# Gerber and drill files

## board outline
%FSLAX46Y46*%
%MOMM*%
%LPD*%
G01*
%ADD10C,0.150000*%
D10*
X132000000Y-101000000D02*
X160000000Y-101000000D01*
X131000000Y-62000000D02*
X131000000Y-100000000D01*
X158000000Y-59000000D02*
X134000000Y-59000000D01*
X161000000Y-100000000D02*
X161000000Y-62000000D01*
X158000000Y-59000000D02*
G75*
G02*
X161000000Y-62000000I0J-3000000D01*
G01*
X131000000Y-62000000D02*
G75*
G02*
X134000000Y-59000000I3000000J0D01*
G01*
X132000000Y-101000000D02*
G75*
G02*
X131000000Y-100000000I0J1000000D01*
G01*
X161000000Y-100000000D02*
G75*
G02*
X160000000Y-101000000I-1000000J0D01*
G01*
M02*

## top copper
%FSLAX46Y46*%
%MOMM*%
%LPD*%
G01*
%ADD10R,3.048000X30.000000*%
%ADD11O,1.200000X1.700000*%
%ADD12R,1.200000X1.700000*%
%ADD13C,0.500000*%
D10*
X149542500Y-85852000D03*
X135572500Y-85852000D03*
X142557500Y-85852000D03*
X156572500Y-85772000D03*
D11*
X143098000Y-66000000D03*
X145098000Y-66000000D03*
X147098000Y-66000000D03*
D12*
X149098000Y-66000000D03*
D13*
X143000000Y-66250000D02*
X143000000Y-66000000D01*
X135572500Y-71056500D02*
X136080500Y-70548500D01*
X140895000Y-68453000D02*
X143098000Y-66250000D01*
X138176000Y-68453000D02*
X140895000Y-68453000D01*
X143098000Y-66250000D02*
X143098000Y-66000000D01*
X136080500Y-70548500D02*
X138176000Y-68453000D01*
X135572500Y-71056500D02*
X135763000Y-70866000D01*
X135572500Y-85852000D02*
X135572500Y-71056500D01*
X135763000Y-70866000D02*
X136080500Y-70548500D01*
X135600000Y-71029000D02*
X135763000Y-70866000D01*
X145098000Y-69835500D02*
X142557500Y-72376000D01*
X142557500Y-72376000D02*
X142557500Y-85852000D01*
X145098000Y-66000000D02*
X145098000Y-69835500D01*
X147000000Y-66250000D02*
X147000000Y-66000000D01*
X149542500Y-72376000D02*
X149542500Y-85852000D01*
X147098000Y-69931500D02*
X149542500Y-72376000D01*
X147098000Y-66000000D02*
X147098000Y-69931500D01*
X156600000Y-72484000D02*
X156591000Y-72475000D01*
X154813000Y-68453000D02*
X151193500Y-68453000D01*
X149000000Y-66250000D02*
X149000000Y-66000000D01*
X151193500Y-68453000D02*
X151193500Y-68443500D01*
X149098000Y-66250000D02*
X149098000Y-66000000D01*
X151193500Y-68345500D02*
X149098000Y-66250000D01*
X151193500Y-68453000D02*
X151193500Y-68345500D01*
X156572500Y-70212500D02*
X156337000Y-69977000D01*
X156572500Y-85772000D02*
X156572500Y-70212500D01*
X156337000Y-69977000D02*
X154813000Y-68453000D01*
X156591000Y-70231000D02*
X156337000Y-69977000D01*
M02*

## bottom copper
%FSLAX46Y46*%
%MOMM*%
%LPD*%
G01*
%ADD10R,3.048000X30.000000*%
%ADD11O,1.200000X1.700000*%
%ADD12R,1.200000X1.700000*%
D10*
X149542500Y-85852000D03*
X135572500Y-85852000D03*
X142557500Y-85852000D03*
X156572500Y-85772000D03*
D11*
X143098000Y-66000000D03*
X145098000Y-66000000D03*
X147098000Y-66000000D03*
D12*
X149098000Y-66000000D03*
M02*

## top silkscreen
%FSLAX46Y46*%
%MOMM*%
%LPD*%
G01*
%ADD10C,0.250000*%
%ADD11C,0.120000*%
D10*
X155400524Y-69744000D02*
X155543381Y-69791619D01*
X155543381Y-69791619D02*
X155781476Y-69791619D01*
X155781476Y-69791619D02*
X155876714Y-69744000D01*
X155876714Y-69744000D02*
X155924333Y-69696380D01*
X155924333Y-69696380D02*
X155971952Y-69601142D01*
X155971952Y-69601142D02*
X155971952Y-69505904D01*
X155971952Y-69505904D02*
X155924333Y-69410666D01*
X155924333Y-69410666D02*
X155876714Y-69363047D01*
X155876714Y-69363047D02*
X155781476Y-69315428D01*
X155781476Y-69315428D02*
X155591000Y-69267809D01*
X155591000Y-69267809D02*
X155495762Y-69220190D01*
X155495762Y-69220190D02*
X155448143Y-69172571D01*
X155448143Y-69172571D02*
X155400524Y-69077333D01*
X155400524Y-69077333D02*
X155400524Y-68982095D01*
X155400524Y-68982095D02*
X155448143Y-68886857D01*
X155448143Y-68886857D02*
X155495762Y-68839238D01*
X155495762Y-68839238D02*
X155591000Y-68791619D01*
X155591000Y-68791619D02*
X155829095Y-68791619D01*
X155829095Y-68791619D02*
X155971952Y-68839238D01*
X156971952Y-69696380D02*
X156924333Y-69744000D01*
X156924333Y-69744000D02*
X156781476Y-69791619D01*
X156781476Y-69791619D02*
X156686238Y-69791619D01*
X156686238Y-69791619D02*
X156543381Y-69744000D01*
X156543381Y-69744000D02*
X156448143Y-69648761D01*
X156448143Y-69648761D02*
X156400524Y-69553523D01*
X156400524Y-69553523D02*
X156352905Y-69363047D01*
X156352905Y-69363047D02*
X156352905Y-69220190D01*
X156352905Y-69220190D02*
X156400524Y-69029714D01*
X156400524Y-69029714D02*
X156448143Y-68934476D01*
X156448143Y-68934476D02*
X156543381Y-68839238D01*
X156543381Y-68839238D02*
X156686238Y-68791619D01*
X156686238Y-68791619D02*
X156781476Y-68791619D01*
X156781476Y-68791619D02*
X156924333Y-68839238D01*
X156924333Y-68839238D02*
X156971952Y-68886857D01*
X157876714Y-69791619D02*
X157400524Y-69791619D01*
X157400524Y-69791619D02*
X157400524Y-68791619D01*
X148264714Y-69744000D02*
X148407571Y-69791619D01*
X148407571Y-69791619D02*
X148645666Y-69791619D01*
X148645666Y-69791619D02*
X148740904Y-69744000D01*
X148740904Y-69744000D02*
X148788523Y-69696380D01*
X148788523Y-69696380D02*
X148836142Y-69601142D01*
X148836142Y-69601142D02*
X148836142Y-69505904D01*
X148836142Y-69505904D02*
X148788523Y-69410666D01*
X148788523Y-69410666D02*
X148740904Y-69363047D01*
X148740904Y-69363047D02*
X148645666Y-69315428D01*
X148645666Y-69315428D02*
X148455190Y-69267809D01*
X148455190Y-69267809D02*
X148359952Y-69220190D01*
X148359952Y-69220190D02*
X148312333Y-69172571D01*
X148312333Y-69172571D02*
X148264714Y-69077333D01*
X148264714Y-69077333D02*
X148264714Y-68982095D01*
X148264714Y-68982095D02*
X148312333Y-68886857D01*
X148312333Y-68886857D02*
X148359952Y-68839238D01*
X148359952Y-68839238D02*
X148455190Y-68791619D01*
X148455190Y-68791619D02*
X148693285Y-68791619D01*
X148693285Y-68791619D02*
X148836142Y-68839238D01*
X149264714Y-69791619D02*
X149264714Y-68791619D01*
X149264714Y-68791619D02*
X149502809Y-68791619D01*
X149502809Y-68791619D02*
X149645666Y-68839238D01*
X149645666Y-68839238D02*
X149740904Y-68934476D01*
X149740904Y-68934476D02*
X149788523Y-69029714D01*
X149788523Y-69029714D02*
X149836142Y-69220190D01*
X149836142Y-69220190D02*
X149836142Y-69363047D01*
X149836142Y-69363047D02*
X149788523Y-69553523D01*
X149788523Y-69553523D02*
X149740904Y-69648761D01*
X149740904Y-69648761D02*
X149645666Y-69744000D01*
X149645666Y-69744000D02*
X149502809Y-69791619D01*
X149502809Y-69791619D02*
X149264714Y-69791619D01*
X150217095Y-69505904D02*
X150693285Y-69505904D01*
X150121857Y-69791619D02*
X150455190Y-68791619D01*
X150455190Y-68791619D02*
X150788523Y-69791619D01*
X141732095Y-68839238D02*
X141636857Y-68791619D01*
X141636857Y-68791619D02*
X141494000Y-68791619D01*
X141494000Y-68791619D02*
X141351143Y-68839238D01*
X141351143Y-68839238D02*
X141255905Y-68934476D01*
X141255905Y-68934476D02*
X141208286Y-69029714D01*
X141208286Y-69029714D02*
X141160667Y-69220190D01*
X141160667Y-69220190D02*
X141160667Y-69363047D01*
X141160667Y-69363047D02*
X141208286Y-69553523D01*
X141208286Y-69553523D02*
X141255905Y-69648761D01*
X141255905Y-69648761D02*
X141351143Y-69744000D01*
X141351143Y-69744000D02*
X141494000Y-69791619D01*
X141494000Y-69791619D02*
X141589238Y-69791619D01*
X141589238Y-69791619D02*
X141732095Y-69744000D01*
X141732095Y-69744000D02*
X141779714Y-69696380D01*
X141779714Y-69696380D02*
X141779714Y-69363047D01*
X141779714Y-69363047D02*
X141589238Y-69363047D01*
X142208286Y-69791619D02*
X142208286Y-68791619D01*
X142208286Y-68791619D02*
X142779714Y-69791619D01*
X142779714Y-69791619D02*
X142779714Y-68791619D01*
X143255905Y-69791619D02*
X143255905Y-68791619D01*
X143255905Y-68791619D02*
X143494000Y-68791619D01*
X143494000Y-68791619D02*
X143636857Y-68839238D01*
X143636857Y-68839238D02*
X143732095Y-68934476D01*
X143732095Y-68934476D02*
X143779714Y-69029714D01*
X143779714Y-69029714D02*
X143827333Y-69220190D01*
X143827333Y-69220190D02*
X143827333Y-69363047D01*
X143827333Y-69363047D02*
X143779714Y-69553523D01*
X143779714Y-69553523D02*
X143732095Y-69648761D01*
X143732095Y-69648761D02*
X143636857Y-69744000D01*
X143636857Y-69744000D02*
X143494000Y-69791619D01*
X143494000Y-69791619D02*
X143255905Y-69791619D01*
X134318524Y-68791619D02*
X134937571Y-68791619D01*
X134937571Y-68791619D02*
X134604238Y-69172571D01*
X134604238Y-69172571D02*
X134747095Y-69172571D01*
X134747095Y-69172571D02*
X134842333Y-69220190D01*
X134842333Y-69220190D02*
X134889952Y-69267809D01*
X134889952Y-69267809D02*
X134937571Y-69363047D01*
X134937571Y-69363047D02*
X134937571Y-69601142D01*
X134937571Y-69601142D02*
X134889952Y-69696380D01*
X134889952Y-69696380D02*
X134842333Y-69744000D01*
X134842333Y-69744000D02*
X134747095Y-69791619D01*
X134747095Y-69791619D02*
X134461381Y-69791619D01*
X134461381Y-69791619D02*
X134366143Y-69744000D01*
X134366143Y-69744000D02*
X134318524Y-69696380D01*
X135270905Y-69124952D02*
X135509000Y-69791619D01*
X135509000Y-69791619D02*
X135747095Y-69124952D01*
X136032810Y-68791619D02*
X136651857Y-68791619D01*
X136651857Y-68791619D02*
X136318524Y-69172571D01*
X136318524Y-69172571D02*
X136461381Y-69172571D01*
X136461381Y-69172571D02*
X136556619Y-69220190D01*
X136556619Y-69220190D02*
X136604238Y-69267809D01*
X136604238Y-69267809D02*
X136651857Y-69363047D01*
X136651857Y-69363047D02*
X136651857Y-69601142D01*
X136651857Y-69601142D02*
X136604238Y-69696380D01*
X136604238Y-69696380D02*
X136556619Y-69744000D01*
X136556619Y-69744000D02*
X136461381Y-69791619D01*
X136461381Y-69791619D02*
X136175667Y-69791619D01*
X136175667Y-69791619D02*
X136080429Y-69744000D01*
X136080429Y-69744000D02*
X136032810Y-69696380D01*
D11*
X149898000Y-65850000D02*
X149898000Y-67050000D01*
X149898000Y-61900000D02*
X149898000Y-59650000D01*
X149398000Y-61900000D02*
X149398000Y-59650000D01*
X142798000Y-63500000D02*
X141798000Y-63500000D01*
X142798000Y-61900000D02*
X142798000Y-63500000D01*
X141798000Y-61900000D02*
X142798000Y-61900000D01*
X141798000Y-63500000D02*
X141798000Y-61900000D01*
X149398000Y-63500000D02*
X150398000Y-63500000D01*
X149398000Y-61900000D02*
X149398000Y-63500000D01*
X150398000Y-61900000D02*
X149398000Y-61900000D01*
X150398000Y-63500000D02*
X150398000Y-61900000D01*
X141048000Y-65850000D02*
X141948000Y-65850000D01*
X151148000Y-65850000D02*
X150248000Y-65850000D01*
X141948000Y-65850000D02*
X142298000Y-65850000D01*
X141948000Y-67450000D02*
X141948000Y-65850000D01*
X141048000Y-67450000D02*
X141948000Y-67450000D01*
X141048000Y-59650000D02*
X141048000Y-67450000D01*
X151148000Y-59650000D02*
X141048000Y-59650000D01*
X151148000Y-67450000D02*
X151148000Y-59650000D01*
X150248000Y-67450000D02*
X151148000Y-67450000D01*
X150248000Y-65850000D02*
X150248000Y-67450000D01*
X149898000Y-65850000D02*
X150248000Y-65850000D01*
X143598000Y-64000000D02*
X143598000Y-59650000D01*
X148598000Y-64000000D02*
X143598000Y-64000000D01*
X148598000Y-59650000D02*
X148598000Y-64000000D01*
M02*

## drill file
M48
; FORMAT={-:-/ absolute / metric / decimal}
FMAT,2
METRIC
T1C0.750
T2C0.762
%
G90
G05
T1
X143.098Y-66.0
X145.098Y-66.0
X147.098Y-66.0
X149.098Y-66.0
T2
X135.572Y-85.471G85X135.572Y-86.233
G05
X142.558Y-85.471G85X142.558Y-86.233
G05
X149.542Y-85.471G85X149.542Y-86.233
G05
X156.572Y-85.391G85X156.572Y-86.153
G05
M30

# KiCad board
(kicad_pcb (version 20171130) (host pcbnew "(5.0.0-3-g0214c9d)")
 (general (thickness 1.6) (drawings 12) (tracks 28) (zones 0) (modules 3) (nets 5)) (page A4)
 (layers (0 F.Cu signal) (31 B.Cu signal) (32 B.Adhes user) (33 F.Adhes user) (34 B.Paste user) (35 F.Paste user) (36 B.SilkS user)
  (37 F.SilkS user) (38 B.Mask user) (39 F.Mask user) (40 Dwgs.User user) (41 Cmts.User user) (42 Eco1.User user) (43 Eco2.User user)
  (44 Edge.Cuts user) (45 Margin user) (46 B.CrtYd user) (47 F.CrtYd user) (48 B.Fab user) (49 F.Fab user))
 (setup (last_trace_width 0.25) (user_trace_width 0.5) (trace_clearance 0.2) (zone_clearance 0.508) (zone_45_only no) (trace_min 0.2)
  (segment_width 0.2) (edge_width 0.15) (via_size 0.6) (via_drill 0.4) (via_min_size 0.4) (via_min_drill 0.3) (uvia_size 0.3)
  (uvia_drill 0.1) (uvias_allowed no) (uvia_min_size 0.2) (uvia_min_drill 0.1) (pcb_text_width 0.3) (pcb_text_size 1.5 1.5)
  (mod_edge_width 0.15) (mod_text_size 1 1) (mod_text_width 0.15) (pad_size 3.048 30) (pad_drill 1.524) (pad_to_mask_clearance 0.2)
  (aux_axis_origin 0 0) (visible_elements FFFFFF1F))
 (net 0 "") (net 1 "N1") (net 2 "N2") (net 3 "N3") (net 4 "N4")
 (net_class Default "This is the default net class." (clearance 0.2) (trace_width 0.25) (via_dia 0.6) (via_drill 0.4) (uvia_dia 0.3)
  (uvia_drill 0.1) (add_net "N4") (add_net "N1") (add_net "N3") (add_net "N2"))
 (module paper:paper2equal (layer B.Cu) (at 145.7325 70.612)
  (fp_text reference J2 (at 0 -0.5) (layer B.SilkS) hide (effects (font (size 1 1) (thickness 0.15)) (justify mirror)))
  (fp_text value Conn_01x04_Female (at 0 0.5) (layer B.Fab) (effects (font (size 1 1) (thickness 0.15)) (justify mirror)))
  (pad 3 thru_hole rect (at 3.81 15.24) (size 3.048 30) (drill oval 0.762 1.524) (layers *.Cu *.Mask) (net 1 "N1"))
  (pad 1 thru_hole rect (at -10.16 15.24) (size 3.048 30) (drill oval 0.762 1.524) (layers *.Cu *.Mask) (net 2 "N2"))
  (pad 2 thru_hole rect (at -3.175 15.24) (size 3.048 30) (drill oval 0.762 1.524) (layers *.Cu *.Mask) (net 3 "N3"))
  (pad 4 thru_hole rect (at 10.84 15.16) (size 3.048 30) (drill oval 0.762 1.524) (layers *.Cu *.Mask) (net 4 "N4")))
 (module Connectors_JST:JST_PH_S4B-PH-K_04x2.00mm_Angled (layer F.Cu) (at 149.098 66 180)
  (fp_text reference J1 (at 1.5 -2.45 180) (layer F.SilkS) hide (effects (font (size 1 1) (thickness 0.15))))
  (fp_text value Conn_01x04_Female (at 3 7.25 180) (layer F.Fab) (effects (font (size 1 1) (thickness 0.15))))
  (fp_line (start -0.8 0.15) (end -0.8 -1.05) (layer F.SilkS) (width 0.12))
  (fp_line (start -0.8 4.1) (end -0.8 6.35) (layer F.SilkS) (width 0.12))
  (fp_line (start -0.3 4.1) (end -0.3 6.35) (layer F.SilkS) (width 0.12))
  (fp_line (start 6.3 2.5) (end 7.3 2.5) (layer F.SilkS) (width 0.12))
  (fp_line (start 6.3 4.1) (end 6.3 2.5) (layer F.SilkS) (width 0.12))
  (fp_line (start 7.3 4.1) (end 6.3 4.1) (layer F.SilkS) (width 0.12))
  (fp_line (start 7.3 2.5) (end 7.3 4.1) (layer F.SilkS) (width 0.12))
  (fp_line (start -0.3 2.5) (end -1.3 2.5) (layer F.SilkS) (width 0.12))
  (fp_line (start -0.3 4.1) (end -0.3 2.5) (layer F.SilkS) (width 0.12))
  (fp_line (start -1.3 4.1) (end -0.3 4.1) (layer F.SilkS) (width 0.12))
  (fp_line (start -1.3 2.5) (end -1.3 4.1) (layer F.SilkS) (width 0.12))
  (fp_line (start 8.05 0.15) (end 7.15 0.15) (layer F.SilkS) (width 0.12))
  (fp_line (start -2.05 0.15) (end -1.15 0.15) (layer F.SilkS) (width 0.12))
  (fp_line (start 7.15 0.15) (end 6.8 0.15) (layer F.SilkS) (width 0.12))
  (fp_line (start 7.15 -1.45) (end 7.15 0.15) (layer F.SilkS) (width 0.12))
  (fp_line (start 8.05 -1.45) (end 7.15 -1.45) (layer F.SilkS) (width 0.12))
  (fp_line (start 8.05 6.35) (end 8.05 -1.45) (layer F.SilkS) (width 0.12))
  (fp_line (start -2.05 6.35) (end 8.05 6.35) (layer F.SilkS) (width 0.12))
  (fp_line (start -2.05 -1.45) (end -2.05 6.35) (layer F.SilkS) (width 0.12))
  (fp_line (start -1.15 -1.45) (end -2.05 -1.45) (layer F.SilkS) (width 0.12))
  (fp_line (start -1.15 0.15) (end -1.15 -1.45) (layer F.SilkS) (width 0.12))
  (fp_line (start -0.8 0.15) (end -1.15 0.15) (layer F.SilkS) (width 0.12))
  (fp_line (start 5.5 2) (end 5.5 6.35) (layer F.SilkS) (width 0.12))
  (fp_line (start 0.5 2) (end 5.5 2) (layer F.SilkS) (width 0.12))
  (fp_line (start 0.5 6.35) (end 0.5 2) (layer F.SilkS) (width 0.12))
  (pad 4 thru_hole oval (at 6 0 180) (size 1.2 1.7) (drill 0.75) (layers *.Cu *.Mask) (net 2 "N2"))
  (pad 3 thru_hole oval (at 4 0 180) (size 1.2 1.7) (drill 0.75) (layers *.Cu *.Mask) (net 3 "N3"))
  (pad 2 thru_hole oval (at 2 0 180) (size 1.2 1.7) (drill 0.75) (layers *.Cu *.Mask) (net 1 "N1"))
  (pad 1 thru_hole rect (at 0 0 180) (size 1.2 1.7) (drill 0.75) (layers *.Cu *.Mask) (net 4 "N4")))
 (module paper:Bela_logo (layer B.Cu) (at 155.067 64.897 135)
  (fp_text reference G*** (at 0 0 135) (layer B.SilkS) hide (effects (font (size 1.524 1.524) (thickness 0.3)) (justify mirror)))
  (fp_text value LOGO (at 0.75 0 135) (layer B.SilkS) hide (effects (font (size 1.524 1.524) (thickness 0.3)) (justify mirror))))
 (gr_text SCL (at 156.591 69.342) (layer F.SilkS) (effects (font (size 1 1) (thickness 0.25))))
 (gr_line (start 132 101) (end 160 101) (angle 90) (layer Edge.Cuts) (width 0.15))
 (gr_line (start 131 62) (end 131 100) (angle 90) (layer Edge.Cuts) (width 0.15))
 (gr_line (start 158 59) (end 134 59) (angle 90) (layer Edge.Cuts) (width 0.15))
 (gr_line (start 161 100) (end 161 62) (angle 90) (layer Edge.Cuts) (width 0.15))
 (gr_arc (start 158 62) (end 158 59) (angle 90) (layer Edge.Cuts) (width 0.15))
 (gr_arc (start 134 62) (end 131 62) (angle 90) (layer Edge.Cuts) (width 0.15))
 (gr_arc (start 132 100) (end 132 101) (angle 90) (layer Edge.Cuts) (width 0.15))
 (gr_arc (start 160 100) (end 161 100) (angle 90) (layer Edge.Cuts) (width 0.15))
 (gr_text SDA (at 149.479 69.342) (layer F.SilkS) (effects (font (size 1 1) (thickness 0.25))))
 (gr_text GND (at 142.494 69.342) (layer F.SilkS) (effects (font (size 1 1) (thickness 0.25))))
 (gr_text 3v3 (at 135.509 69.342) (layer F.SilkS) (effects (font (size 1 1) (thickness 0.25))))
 (segment (start 143 66.25) (end 143 66) (width 0.5) (layer F.Cu) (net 2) (status 30))
 (segment (start 135.5725 71.0565) (end 136.0805 70.5485) (width 0.5) (layer F.Cu) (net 2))
 (segment (start 140.895 68.453) (end 143.098 66.25) (width 0.5) (layer F.Cu) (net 2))
 (segment (start 138.176 68.453) (end 140.895 68.453) (width 0.5) (layer F.Cu) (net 2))
 (segment (start 143.098 66.25) (end 143.098 66) (width 0.5) (layer F.Cu) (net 2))
 (segment (start 136.0805 70.5485) (end 138.176 68.453) (width 0.5) (layer F.Cu) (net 2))
 (segment (start 135.5725 71.0565) (end 135.763 70.866) (width 0.5) (layer F.Cu) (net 2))
 (segment (start 135.5725 85.852) (end 135.5725 71.0565) (width 0.5) (layer F.Cu) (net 2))
 (segment (start 135.763 70.866) (end 136.0805 70.5485) (width 0.5) (layer F.Cu) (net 2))
 (segment (start 135.6 71.029) (end 135.763 70.866) (width 0.5) (layer F.Cu) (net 2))
 (segment (start 145.098 69.8355) (end 142.5575 72.376) (width 0.5) (layer F.Cu) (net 3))
 (segment (start 142.5575 72.376) (end 142.5575 85.852) (width 0.5) (layer F.Cu) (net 3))
 (segment (start 145.098 66) (end 145.098 69.8355) (width 0.5) (layer F.Cu) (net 3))
 (segment (start 147 66.25) (end 147 66) (width 0.5) (layer F.Cu) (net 1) (status 30))
 (segment (start 149.5425 72.376) (end 149.5425 85.852) (width 0.5) (layer F.Cu) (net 1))
 (segment (start 147.098 69.9315) (end 149.5425 72.376) (width 0.5) (layer F.Cu) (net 1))
 (segment (start 147.098 66) (end 147.098 69.9315) (width 0.5) (layer F.Cu) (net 1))
 (segment (start 156.6 72.484) (end 156.591 72.475) (width 0.5) (layer F.Cu) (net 4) (status 30))
 (segment (start 154.813 68.453) (end 151.1935 68.453) (width 0.5) (layer F.Cu) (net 4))
 (segment (start 149 66.25) (end 149 66) (width 0.5) (layer F.Cu) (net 4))
 (segment (start 151.1935 68.453) (end 151.1935 68.4435) (width 0.5) (layer F.Cu) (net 4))
 (segment (start 149.098 66.25) (end 149.098 66) (width 0.5) (layer F.Cu) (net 4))
 (segment (start 151.1935 68.3455) (end 149.098 66.25) (width 0.5) (layer F.Cu) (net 4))
 (segment (start 151.1935 68.453) (end 151.1935 68.3455) (width 0.5) (layer F.Cu) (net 4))
 (segment (start 156.5725 70.2125) (end 156.337 69.977) (width 0.5) (layer F.Cu) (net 4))
 (segment (start 156.5725 85.772) (end 156.5725 70.2125) (width 0.5) (layer F.Cu) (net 4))
 (segment (start 156.337 69.977) (end 154.813 68.453) (width 0.5) (layer F.Cu) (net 4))
 (segment (start 156.591 70.231) (end 156.337 69.977) (width 0.5) (layer F.Cu) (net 4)))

